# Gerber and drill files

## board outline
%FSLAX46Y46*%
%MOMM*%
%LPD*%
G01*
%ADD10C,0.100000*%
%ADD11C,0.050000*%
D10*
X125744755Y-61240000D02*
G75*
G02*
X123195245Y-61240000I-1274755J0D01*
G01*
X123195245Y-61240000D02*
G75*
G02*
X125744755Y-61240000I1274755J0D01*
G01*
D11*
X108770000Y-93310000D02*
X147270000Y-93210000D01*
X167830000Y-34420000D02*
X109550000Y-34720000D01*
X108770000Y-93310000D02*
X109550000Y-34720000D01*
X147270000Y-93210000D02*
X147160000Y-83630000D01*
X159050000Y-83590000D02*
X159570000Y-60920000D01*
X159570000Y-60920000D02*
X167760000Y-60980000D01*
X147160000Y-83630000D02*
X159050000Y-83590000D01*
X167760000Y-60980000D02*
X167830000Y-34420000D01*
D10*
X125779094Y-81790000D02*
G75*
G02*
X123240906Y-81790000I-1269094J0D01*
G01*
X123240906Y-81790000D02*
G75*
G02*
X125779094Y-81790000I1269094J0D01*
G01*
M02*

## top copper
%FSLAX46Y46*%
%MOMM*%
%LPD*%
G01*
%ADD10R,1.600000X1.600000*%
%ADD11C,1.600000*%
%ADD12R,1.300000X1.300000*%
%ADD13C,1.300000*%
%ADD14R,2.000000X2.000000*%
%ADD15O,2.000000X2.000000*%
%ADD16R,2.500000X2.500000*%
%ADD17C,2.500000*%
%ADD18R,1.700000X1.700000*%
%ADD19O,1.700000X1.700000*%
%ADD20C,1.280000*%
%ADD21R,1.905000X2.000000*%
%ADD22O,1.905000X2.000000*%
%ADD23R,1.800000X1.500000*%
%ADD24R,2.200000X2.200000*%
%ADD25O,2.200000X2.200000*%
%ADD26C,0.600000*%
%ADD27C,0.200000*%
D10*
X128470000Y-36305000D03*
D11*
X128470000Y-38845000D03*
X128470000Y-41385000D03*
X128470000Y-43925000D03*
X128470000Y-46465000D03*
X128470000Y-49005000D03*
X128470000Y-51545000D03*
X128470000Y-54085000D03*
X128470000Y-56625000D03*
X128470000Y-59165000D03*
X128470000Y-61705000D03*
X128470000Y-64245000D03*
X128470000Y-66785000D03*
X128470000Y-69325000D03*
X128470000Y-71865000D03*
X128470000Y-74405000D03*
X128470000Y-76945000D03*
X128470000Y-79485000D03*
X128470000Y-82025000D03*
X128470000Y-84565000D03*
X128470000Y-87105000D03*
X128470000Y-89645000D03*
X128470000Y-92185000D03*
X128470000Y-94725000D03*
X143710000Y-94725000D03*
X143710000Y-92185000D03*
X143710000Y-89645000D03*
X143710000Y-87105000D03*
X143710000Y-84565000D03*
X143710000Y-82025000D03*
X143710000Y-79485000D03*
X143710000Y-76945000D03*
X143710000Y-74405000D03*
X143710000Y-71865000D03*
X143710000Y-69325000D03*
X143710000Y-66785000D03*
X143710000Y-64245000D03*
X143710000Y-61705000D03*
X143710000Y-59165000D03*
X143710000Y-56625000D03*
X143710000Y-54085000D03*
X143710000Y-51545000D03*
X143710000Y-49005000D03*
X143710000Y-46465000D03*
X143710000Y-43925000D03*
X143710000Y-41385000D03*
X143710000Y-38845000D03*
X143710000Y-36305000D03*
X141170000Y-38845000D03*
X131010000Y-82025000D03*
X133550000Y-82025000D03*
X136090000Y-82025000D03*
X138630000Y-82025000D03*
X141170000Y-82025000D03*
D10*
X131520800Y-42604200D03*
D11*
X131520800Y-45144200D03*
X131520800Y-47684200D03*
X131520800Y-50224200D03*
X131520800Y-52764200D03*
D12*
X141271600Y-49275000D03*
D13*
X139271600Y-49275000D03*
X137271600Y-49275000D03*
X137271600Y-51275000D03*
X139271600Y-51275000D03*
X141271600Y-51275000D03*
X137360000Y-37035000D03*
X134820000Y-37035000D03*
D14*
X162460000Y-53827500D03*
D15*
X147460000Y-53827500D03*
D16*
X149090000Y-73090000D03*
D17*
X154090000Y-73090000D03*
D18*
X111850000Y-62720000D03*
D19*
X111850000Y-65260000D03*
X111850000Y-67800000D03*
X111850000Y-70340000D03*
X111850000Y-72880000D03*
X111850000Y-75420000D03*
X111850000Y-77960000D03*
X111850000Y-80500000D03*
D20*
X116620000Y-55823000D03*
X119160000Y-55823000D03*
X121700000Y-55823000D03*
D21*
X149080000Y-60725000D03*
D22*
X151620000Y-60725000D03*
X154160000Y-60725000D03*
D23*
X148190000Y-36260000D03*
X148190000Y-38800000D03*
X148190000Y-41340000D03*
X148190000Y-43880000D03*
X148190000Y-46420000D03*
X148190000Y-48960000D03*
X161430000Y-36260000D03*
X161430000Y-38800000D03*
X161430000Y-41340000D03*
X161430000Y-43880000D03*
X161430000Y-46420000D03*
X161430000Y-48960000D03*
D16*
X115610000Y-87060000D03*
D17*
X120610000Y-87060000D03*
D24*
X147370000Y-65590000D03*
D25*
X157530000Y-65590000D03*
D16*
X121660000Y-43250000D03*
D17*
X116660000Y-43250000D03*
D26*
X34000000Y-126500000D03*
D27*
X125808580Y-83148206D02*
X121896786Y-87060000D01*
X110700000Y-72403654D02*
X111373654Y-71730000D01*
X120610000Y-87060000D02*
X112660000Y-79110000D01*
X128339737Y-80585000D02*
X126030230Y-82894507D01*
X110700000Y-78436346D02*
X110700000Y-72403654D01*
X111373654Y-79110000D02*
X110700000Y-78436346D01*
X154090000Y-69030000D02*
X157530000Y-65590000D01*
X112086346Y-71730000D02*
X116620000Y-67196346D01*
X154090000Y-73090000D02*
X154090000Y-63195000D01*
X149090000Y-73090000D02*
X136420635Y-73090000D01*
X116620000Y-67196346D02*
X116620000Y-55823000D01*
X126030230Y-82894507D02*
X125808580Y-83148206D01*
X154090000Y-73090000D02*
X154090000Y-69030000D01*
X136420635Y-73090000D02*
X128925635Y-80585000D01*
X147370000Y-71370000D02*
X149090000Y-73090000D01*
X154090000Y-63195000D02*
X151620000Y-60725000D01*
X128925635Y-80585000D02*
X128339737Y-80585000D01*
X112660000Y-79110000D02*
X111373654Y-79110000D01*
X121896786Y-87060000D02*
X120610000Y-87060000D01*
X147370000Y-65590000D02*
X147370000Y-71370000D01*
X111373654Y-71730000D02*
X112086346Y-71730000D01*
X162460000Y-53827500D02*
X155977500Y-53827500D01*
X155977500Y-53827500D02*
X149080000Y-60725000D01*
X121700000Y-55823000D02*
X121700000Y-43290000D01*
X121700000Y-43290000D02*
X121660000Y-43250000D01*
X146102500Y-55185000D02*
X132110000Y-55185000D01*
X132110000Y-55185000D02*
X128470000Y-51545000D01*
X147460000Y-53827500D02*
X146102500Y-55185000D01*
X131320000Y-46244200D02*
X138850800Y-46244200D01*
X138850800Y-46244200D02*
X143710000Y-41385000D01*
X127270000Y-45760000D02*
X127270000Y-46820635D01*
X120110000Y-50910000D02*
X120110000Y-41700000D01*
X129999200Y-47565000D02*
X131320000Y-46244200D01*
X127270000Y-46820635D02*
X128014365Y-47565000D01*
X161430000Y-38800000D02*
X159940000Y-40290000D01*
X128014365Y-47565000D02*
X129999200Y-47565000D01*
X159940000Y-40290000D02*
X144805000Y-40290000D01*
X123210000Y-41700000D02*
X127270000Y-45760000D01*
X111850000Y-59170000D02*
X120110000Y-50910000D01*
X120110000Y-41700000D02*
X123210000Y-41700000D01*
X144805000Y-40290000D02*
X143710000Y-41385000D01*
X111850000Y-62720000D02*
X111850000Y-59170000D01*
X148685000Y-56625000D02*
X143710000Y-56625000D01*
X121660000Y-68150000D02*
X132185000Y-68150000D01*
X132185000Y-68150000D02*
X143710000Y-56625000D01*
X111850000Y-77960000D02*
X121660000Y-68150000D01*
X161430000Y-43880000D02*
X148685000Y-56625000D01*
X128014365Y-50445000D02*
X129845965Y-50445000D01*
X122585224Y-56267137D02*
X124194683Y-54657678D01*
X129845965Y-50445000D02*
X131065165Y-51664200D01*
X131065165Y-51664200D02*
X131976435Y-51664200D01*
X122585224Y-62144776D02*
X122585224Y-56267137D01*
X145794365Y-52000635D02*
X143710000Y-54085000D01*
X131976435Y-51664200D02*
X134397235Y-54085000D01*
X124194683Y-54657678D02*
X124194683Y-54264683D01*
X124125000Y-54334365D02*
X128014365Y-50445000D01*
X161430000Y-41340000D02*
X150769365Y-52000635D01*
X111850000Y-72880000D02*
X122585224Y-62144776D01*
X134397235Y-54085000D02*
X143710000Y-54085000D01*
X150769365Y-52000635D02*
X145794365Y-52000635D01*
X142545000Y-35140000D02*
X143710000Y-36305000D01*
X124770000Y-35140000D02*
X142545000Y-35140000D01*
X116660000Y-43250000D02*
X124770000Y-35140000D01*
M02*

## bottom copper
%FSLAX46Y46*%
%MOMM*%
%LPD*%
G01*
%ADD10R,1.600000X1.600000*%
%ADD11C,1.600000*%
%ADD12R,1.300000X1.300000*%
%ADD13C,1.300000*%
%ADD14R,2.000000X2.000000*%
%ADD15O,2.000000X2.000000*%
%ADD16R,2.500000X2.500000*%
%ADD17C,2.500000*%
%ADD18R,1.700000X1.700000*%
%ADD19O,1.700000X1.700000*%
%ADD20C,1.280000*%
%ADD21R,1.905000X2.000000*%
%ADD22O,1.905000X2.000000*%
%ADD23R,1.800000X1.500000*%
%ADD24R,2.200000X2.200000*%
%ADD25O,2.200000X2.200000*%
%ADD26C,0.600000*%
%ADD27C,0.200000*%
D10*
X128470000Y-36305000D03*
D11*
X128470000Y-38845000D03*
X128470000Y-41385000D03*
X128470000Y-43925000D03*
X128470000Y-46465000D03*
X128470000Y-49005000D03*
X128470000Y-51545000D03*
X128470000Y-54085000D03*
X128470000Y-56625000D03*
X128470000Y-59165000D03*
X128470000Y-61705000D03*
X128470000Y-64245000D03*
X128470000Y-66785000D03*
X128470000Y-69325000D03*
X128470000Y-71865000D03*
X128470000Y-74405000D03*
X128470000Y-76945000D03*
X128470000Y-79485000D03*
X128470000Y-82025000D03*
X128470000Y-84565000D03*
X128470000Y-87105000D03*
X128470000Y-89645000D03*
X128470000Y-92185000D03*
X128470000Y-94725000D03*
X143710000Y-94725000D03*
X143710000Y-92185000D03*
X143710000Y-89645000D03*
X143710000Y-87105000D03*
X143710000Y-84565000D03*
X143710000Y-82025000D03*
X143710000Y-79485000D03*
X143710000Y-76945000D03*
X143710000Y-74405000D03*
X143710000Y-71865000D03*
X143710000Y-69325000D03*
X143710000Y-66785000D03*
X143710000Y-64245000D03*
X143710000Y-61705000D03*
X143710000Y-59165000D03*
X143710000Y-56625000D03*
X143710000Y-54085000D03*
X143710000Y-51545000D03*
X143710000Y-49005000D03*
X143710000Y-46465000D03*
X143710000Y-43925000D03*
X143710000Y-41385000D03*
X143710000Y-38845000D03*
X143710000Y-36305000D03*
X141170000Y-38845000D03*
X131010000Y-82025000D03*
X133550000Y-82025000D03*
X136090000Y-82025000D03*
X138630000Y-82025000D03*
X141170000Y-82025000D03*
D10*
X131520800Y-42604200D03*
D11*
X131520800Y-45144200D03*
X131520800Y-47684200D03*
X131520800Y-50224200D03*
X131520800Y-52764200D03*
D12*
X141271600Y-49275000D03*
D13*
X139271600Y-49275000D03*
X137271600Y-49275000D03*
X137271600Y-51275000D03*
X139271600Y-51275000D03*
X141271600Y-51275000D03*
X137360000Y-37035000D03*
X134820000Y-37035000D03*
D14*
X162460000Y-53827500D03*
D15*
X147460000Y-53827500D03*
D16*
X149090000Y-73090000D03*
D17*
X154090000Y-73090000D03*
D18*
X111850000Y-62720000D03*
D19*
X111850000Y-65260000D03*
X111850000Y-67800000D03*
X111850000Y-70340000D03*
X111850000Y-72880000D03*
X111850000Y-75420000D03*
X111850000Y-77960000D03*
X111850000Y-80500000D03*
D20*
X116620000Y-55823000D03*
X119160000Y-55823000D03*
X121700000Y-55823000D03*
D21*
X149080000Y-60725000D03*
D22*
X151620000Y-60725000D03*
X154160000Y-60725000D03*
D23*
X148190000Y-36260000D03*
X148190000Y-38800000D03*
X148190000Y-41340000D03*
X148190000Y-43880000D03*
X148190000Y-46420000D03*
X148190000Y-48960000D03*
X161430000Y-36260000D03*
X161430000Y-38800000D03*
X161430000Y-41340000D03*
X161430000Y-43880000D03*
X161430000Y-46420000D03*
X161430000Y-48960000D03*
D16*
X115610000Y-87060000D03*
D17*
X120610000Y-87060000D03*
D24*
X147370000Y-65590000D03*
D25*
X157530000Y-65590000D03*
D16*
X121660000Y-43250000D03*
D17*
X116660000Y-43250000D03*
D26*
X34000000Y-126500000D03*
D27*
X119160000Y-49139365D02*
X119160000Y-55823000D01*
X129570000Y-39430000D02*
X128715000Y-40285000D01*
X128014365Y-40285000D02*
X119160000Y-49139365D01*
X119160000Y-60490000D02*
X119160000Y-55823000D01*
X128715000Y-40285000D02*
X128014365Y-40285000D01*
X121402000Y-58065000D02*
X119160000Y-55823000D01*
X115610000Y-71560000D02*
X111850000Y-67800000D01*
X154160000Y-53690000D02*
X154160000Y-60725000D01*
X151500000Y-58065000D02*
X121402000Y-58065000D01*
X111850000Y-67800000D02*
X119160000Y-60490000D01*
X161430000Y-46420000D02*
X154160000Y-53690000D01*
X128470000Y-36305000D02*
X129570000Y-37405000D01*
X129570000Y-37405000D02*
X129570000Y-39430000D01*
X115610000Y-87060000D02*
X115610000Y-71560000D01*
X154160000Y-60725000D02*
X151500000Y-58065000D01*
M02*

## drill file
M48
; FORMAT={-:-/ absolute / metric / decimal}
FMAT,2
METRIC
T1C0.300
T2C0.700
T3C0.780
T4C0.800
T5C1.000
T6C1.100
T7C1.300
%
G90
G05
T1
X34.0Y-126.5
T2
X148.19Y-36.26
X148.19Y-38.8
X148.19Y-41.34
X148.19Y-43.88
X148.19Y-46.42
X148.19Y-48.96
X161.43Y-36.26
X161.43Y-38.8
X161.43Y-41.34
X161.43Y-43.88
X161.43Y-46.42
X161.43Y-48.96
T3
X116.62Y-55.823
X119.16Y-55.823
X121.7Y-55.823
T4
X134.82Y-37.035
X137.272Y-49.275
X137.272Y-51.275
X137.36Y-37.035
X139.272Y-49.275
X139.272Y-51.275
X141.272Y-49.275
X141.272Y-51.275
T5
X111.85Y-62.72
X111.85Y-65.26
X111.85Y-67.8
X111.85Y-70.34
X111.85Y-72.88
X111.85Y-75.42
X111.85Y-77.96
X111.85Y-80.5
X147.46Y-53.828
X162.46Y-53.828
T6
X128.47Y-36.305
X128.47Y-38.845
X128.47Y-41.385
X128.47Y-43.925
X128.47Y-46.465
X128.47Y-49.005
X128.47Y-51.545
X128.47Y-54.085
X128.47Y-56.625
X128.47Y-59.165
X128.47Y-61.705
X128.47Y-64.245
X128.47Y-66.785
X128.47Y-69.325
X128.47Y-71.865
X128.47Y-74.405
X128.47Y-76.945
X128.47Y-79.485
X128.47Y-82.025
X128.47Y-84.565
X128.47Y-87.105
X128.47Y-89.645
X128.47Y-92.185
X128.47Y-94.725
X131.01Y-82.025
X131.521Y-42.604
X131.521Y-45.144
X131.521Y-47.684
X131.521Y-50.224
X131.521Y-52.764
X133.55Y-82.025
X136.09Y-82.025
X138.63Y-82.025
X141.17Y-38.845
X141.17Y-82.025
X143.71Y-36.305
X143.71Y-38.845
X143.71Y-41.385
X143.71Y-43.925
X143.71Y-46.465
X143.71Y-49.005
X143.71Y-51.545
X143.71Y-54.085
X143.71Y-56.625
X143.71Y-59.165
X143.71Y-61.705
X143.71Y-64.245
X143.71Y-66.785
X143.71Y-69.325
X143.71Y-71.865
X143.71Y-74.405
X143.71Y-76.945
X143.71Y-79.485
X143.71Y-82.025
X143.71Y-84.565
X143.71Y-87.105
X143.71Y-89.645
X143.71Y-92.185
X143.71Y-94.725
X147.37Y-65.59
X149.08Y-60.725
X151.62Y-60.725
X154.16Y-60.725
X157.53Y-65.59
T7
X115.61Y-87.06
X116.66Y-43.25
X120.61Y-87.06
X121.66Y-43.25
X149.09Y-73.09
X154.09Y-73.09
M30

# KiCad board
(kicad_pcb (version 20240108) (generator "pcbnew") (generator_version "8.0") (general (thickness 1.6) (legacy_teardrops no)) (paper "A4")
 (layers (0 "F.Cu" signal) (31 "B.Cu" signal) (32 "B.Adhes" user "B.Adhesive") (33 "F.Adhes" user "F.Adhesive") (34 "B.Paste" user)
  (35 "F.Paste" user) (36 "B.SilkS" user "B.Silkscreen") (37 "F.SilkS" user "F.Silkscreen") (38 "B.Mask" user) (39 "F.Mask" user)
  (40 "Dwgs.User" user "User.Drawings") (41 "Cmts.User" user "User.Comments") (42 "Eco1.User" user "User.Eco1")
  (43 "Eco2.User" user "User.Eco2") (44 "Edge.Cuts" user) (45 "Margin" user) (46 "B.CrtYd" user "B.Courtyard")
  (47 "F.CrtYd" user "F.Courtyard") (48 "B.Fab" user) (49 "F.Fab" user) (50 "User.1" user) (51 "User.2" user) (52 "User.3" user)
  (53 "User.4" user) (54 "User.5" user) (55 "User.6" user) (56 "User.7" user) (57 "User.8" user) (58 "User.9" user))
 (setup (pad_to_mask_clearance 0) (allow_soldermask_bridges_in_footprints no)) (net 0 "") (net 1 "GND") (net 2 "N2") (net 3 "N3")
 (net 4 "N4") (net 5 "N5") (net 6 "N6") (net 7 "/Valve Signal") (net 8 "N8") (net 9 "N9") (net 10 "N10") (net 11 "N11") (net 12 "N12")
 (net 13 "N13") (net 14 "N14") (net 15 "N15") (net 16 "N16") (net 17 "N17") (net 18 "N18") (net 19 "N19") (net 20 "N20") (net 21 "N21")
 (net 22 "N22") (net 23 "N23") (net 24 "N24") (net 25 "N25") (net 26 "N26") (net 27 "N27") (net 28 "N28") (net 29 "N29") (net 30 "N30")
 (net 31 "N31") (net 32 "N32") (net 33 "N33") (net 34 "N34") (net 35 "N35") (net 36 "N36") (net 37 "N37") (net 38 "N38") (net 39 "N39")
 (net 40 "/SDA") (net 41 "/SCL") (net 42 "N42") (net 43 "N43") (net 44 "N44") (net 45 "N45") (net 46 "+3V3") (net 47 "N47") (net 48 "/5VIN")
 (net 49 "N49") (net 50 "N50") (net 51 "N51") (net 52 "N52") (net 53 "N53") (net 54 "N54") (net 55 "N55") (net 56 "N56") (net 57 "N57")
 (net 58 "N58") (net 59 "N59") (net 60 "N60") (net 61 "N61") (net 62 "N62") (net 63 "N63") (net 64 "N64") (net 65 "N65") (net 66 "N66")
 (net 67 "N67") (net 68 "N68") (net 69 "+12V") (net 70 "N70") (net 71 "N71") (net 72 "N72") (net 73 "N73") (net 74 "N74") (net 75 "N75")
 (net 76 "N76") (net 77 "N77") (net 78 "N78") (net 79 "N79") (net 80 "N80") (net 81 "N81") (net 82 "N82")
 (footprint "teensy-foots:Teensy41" (layer "F.Cu") (at 136.09 65.515 -90)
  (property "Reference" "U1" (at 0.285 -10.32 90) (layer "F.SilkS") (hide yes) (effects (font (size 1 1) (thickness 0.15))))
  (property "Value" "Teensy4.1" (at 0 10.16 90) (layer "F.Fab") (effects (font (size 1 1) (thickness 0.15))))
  (pad "1" thru_hole rect (at -29.21 7.62 270) (size 1.6 1.6) (drill 1.1) (layers "*.Cu" "*.Mask") (remove_unused_layers no) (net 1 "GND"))
  (pad "2" thru_hole circle (at -26.67 7.62 270) (size 1.6 1.6) (drill 1.1) (layers "*.Cu" "*.Mask") (remove_unused_layers no) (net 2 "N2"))
  (pad "3" thru_hole circle (at -24.13 7.62 270) (size 1.6 1.6) (drill 1.1) (layers "*.Cu" "*.Mask") (remove_unused_layers no) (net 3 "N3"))
  (pad "4" thru_hole circle (at -21.59 7.62 270) (size 1.6 1.6) (drill 1.1) (layers "*.Cu" "*.Mask") (remove_unused_layers no) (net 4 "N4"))
  (pad "5" thru_hole circle (at -19.05 7.62 270) (size 1.6 1.6) (drill 1.1) (layers "*.Cu" "*.Mask") (remove_unused_layers no) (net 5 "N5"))
  (pad "6" thru_hole circle (at -16.51 7.62 270) (size 1.6 1.6) (drill 1.1) (layers "*.Cu" "*.Mask") (remove_unused_layers no) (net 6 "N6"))
  (pad "7" thru_hole circle (at -13.97 7.62 270) (size 1.6 1.6) (drill 1.1) (layers "*.Cu" "*.Mask") (remove_unused_layers no)
   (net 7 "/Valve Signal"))
  (pad "8" thru_hole circle (at -11.43 7.62 270) (size 1.6 1.6) (drill 1.1) (layers "*.Cu" "*.Mask") (remove_unused_layers no) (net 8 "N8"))
  (pad "9" thru_hole circle (at -8.89 7.62 270) (size 1.6 1.6) (drill 1.1) (layers "*.Cu" "*.Mask") (remove_unused_layers no) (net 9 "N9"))
  (pad "10" thru_hole circle (at -6.35 7.62 270) (size 1.6 1.6) (drill 1.1) (layers "*.Cu" "*.Mask") (remove_unused_layers no)
   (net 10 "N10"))
  (pad "11" thru_hole circle (at -3.81 7.62 270) (size 1.6 1.6) (drill 1.1) (layers "*.Cu" "*.Mask") (remove_unused_layers no)
   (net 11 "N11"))
  (pad "12" thru_hole circle (at -1.27 7.62 270) (size 1.6 1.6) (drill 1.1) (layers "*.Cu" "*.Mask") (remove_unused_layers no)
   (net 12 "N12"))
  (pad "13" thru_hole circle (at 1.27 7.62 270) (size 1.6 1.6) (drill 1.1) (layers "*.Cu" "*.Mask") (remove_unused_layers no) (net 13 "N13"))
  (pad "14" thru_hole circle (at 3.81 7.62 270) (size 1.6 1.6) (drill 1.1) (layers "*.Cu" "*.Mask") (remove_unused_layers no) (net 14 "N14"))
  (pad "15" thru_hole circle (at 6.35 7.62 270) (size 1.6 1.6) (drill 1.1) (layers "*.Cu" "*.Mask") (remove_unused_layers no) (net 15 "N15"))
  (pad "16" thru_hole circle (at 8.89 7.62 270) (size 1.6 1.6) (drill 1.1) (layers "*.Cu" "*.Mask") (remove_unused_layers no) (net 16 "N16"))
  (pad "17" thru_hole circle (at 11.43 7.62 270) (size 1.6 1.6) (drill 1.1) (layers "*.Cu" "*.Mask") (remove_unused_layers no)
   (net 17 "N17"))
  (pad "18" thru_hole circle (at 13.97 7.62 270) (size 1.6 1.6) (drill 1.1) (layers "*.Cu" "*.Mask") (remove_unused_layers no)
   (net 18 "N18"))
  (pad "19" thru_hole circle (at 16.51 7.62 270) (size 1.6 1.6) (drill 1.1) (layers "*.Cu" "*.Mask") (remove_unused_layers no)
   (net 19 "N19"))
  (pad "20" thru_hole circle (at 19.05 7.62 270) (size 1.6 1.6) (drill 1.1) (layers "*.Cu" "*.Mask") (remove_unused_layers no)
   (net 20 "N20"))
  (pad "21" thru_hole circle (at 21.59 7.62 270) (size 1.6 1.6) (drill 1.1) (layers "*.Cu" "*.Mask") (remove_unused_layers no)
   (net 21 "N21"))
  (pad "22" thru_hole circle (at 24.13 7.62 270) (size 1.6 1.6) (drill 1.1) (layers "*.Cu" "*.Mask") (remove_unused_layers no)
   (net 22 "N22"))
  (pad "23" thru_hole circle (at 26.67 7.62 270) (size 1.6 1.6) (drill 1.1) (layers "*.Cu" "*.Mask") (remove_unused_layers no)
   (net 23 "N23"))
  (pad "24" thru_hole circle (at 29.21 7.62 270) (size 1.6 1.6) (drill 1.1) (layers "*.Cu" "*.Mask") (remove_unused_layers no)
   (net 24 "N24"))
  (pad "25" thru_hole circle (at 29.21 -7.62 270) (size 1.6 1.6) (drill 1.1) (layers "*.Cu" "*.Mask") (remove_unused_layers no)
   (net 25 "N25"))
  (pad "26" thru_hole circle (at 26.67 -7.62 270) (size 1.6 1.6) (drill 1.1) (layers "*.Cu" "*.Mask") (remove_unused_layers no)
   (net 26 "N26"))
  (pad "27" thru_hole circle (at 24.13 -7.62 270) (size 1.6 1.6) (drill 1.1) (layers "*.Cu" "*.Mask") (remove_unused_layers no)
   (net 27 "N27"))
  (pad "28" thru_hole circle (at 21.59 -7.62 270) (size 1.6 1.6) (drill 1.1) (layers "*.Cu" "*.Mask") (remove_unused_layers no)
   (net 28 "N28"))
  (pad "29" thru_hole circle (at 19.05 -7.62 270) (size 1.6 1.6) (drill 1.1) (layers "*.Cu" "*.Mask") (remove_unused_layers no)
   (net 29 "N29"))
  (pad "30" thru_hole circle (at 16.51 -7.62 270) (size 1.6 1.6) (drill 1.1) (layers "*.Cu" "*.Mask") (remove_unused_layers no)
   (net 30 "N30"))
  (pad "31" thru_hole circle (at 13.97 -7.62 270) (size 1.6 1.6) (drill 1.1) (layers "*.Cu" "*.Mask") (remove_unused_layers no)
   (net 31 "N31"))
  (pad "32" thru_hole circle (at 11.43 -7.62 270) (size 1.6 1.6) (drill 1.1) (layers "*.Cu" "*.Mask") (remove_unused_layers no)
   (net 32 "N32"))
  (pad "33" thru_hole circle (at 8.89 -7.62 270) (size 1.6 1.6) (drill 1.1) (layers "*.Cu" "*.Mask") (remove_unused_layers no)
   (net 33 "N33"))
  (pad "34" thru_hole circle (at 6.35 -7.62 270) (size 1.6 1.6) (drill 1.1) (layers "*.Cu" "*.Mask") (remove_unused_layers no)
   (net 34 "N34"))
  (pad "35" thru_hole circle (at 3.81 -7.62 270) (size 1.6 1.6) (drill 1.1) (layers "*.Cu" "*.Mask") (remove_unused_layers no)
   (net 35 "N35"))
  (pad "36" thru_hole circle (at 1.27 -7.62 270) (size 1.6 1.6) (drill 1.1) (layers "*.Cu" "*.Mask") (remove_unused_layers no)
   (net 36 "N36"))
  (pad "37" thru_hole circle (at -1.27 -7.62 270) (size 1.6 1.6) (drill 1.1) (layers "*.Cu" "*.Mask") (remove_unused_layers no)
   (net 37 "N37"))
  (pad "38" thru_hole circle (at -3.81 -7.62 270) (size 1.6 1.6) (drill 1.1) (layers "*.Cu" "*.Mask") (remove_unused_layers no)
   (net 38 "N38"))
  (pad "39" thru_hole circle (at -6.35 -7.62 270) (size 1.6 1.6) (drill 1.1) (layers "*.Cu" "*.Mask") (remove_unused_layers no)
   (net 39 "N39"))
  (pad "40" thru_hole circle (at -8.89 -7.62 270) (size 1.6 1.6) (drill 1.1) (layers "*.Cu" "*.Mask") (remove_unused_layers no)
   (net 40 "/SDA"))
  (pad "41" thru_hole circle (at -11.43 -7.62 270) (size 1.6 1.6) (drill 1.1) (layers "*.Cu" "*.Mask") (remove_unused_layers no)
   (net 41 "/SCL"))
  (pad "42" thru_hole circle (at -13.97 -7.62 270) (size 1.6 1.6) (drill 1.1) (layers "*.Cu" "*.Mask") (remove_unused_layers no)
   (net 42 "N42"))
  (pad "43" thru_hole circle (at -16.51 -7.62 270) (size 1.6 1.6) (drill 1.1) (layers "*.Cu" "*.Mask") (remove_unused_layers no)
   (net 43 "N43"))
  (pad "44" thru_hole circle (at -19.05 -7.62 270) (size 1.6 1.6) (drill 1.1) (layers "*.Cu" "*.Mask") (remove_unused_layers no)
   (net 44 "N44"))
  (pad "45" thru_hole circle (at -21.59 -7.62 270) (size 1.6 1.6) (drill 1.1) (layers "*.Cu" "*.Mask") (remove_unused_layers no)
   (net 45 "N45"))
  (pad "46" thru_hole circle (at -24.13 -7.62 270) (size 1.6 1.6) (drill 1.1) (layers "*.Cu" "*.Mask") (remove_unused_layers no)
   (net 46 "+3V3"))
  (pad "47" thru_hole circle (at -26.67 -7.62 270) (size 1.6 1.6) (drill 1.1) (layers "*.Cu" "*.Mask") (remove_unused_layers no)
   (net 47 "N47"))
  (pad "48" thru_hole circle (at -29.21 -7.62 270) (size 1.6 1.6) (drill 1.1) (layers "*.Cu" "*.Mask") (remove_unused_layers no)
   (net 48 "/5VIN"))
  (pad "49" thru_hole circle (at -26.67 -5.08 270) (size 1.6 1.6) (drill 1.1) (layers "*.Cu" "*.Mask") (remove_unused_layers no)
   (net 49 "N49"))
  (pad "50" thru_hole circle (at 16.51 5.08 270) (size 1.6 1.6) (drill 1.1) (layers "*.Cu" "*.Mask") (remove_unused_layers no)
   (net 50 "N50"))
  (pad "51" thru_hole circle (at 16.51 2.54 270) (size 1.6 1.6) (drill 1.1) (layers "*.Cu" "*.Mask") (remove_unused_layers no)
   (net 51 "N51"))
  (pad "52" thru_hole circle (at 16.51 0 270) (size 1.6 1.6) (drill 1.1) (layers "*.Cu" "*.Mask") (remove_unused_layers no) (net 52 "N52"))
  (pad "53" thru_hole circle (at 16.51 -2.54 270) (size 1.6 1.6) (drill 1.1) (layers "*.Cu" "*.Mask") (remove_unused_layers no)
   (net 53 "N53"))
  (pad "54" thru_hole circle (at 16.51 -5.08 270) (size 1.6 1.6) (drill 1.1) (layers "*.Cu" "*.Mask") (remove_unused_layers no)
   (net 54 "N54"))
  (pad "55" thru_hole rect (at -22.9108 4.5692 270) (size 1.6 1.6) (drill 1.1) (layers "*.Cu" "*.Mask") (remove_unused_layers no)
   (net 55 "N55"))
  (pad "56" thru_hole circle (at -20.3708 4.5692 270) (size 1.6 1.6) (drill 1.1) (layers "*.Cu" "*.Mask") (remove_unused_layers no)
   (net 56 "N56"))
  (pad "57" thru_hole circle (at -17.8308 4.5692 270) (size 1.6 1.6) (drill 1.1) (layers "*.Cu" "*.Mask") (remove_unused_layers no)
   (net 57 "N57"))
  (pad "58" thru_hole circle (at -15.2908 4.5692 270) (size 1.6 1.6) (drill 1.1) (layers "*.Cu" "*.Mask") (remove_unused_layers no)
   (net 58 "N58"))
  (pad "59" thru_hole circle (at -12.7508 4.5692 270) (size 1.6 1.6) (drill 1.1) (layers "*.Cu" "*.Mask") (remove_unused_layers no)
   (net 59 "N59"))
  (pad "60" thru_hole rect (at -16.24 -5.1816 270) (size 1.3 1.3) (drill 0.8) (layers "*.Cu" "*.Mask") (remove_unused_layers no)
   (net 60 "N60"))
  (pad "61" thru_hole circle (at -16.24 -3.1816 270) (size 1.3 1.3) (drill 0.8) (layers "*.Cu" "*.Mask") (remove_unused_layers no)
   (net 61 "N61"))
  (pad "62" thru_hole circle (at -16.24 -1.1816 270) (size 1.3 1.3) (drill 0.8) (layers "*.Cu" "*.Mask") (remove_unused_layers no)
   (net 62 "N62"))
  (pad "63" thru_hole circle (at -14.24 -1.1816 270) (size 1.3 1.3) (drill 0.8) (layers "*.Cu" "*.Mask") (remove_unused_layers no)
   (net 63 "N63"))
  (pad "64" thru_hole circle (at -14.24 -3.1816 270) (size 1.3 1.3) (drill 0.8) (layers "*.Cu" "*.Mask") (remove_unused_layers no)
   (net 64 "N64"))
  (pad "65" thru_hole circle (at -14.24 -5.1816 270) (size 1.3 1.3) (drill 0.8) (layers "*.Cu" "*.Mask") (remove_unused_layers no)
   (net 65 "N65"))
  (pad "66" thru_hole circle (at -28.48 -1.27 270) (size 1.3 1.3) (drill 0.8) (layers "*.Cu" "*.Mask") (remove_unused_layers no)
   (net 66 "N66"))
  (pad "67" thru_hole circle (at -28.48 1.27 270) (size 1.3 1.3) (drill 0.8) (layers "*.Cu" "*.Mask") (remove_unused_layers no)
   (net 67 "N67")))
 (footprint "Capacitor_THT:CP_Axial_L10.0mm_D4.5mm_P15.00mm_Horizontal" (layer "F.Cu") (at 162.46 53.8275 180)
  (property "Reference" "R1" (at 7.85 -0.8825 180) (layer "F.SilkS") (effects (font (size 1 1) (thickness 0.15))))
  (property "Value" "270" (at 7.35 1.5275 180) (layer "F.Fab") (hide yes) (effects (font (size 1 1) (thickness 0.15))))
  (pad "1" thru_hole rect (at 0 0 180) (size 2 2) (drill 1) (layers "*.Cu" "*.Mask") (remove_unused_layers no) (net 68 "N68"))
  (pad "2" thru_hole oval (at 15 0 180) (size 2 2) (drill 1) (layers "*.Cu" "*.Mask") (remove_unused_layers no) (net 7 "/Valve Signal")))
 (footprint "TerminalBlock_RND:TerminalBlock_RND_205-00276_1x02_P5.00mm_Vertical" (layer "F.Cu") (at 149.09 73.09)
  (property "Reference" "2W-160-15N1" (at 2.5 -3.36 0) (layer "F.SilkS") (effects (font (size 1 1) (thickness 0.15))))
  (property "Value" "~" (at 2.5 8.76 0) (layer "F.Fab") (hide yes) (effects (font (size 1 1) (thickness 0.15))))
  (pad "1" thru_hole rect (at 0 0) (size 2.5 2.5) (drill 1.3) (layers "*.Cu" "*.Mask") (remove_unused_layers no) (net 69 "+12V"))
  (pad "2" thru_hole circle (at 5 0) (size 2.5 2.5) (drill 1.3) (layers "*.Cu" "*.Mask") (remove_unused_layers no) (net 69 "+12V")))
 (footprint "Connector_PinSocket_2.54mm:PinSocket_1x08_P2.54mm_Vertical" (layer "F.Cu") (at 111.85 62.72)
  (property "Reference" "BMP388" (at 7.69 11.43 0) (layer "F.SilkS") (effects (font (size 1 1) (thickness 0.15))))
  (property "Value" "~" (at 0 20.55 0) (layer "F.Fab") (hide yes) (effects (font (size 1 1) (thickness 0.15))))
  (pad "1" thru_hole rect (at 0 0) (size 1.7 1.7) (drill 1) (layers "*.Cu" "*.Mask") (remove_unused_layers no) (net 46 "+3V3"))
  (pad "2" thru_hole oval (at 0 2.54) (size 1.7 1.7) (drill 1) (layers "*.Cu" "*.Mask") (remove_unused_layers no) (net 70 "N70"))
  (pad "3" thru_hole oval (at 0 5.08) (size 1.7 1.7) (drill 1) (layers "*.Cu" "*.Mask") (remove_unused_layers no) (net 1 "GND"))
  (pad "4" thru_hole oval (at 0 7.62) (size 1.7 1.7) (drill 1) (layers "*.Cu" "*.Mask") (remove_unused_layers no) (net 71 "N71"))
  (pad "5" thru_hole oval (at 0 10.16) (size 1.7 1.7) (drill 1) (layers "*.Cu" "*.Mask") (remove_unused_layers no) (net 41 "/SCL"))
  (pad "6" thru_hole oval (at 0 12.7) (size 1.7 1.7) (drill 1) (layers "*.Cu" "*.Mask") (remove_unused_layers no) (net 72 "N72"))
  (pad "7" thru_hole oval (at 0 15.24) (size 1.7 1.7) (drill 1) (layers "*.Cu" "*.Mask") (remove_unused_layers no) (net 40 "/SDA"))
  (pad "8" thru_hole oval (at 0 17.78) (size 1.7 1.7) (drill 1) (layers "*.Cu" "*.Mask") (remove_unused_layers no) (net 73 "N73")))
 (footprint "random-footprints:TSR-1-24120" (layer "F.Cu") (at 119.16 55.823)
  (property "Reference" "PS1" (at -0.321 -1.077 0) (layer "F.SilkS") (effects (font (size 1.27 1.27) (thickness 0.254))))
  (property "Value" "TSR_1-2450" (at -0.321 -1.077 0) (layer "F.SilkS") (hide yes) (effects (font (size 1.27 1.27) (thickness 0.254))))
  (pad "1" thru_hole circle (at -2.54 0) (size 1.28 1.28) (drill 0.78) (layers "*.Cu" "*.Mask") (remove_unused_layers no) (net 69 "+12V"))
  (pad "2" thru_hole circle (at 0 0) (size 1.28 1.28) (drill 0.78) (layers "*.Cu" "*.Mask") (remove_unused_layers no) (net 1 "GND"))
  (pad "3" thru_hole circle (at 2.54 0) (size 1.28 1.28) (drill 0.78) (layers "*.Cu" "*.Mask") (remove_unused_layers no) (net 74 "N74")))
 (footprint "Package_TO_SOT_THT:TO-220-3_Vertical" (layer "F.Cu") (at 149.08 60.725)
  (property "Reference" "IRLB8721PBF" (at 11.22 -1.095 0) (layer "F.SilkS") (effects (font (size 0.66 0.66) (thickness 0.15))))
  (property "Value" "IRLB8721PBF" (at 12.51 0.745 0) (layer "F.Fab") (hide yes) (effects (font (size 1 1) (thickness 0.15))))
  (pad "1" thru_hole rect (at 0 0) (size 1.905 2) (drill 1.1) (layers "*.Cu" "*.Mask") (remove_unused_layers no) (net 68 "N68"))
  (pad "2" thru_hole oval (at 2.54 0) (size 1.905 2) (drill 1.1) (layers "*.Cu" "*.Mask") (remove_unused_layers no) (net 69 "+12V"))
  (pad "3" thru_hole oval (at 5.08 0) (size 1.905 2) (drill 1.1) (layers "*.Cu" "*.Mask") (remove_unused_layers no) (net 1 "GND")))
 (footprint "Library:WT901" (layer "F.Cu") (at 147.19 34.99)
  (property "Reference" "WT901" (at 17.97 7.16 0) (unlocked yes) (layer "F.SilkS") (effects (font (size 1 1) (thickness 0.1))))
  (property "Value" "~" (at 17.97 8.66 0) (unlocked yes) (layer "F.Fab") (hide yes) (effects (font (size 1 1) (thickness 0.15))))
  (pad "1" thru_hole rect (at 1 1.27) (size 1.8 1.5) (drill 0.7) (layers "*.Cu" "*.Mask") (remove_unused_layers no) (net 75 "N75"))
  (pad "2" thru_hole rect (at 1 3.81) (size 1.8 1.5) (drill 0.7) (layers "*.Cu" "*.Mask") (remove_unused_layers no) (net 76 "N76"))
  (pad "3" thru_hole rect (at 1 6.35) (size 1.8 1.5) (drill 0.7) (layers "*.Cu" "*.Mask") (remove_unused_layers no) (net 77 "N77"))
  (pad "4" thru_hole rect (at 1 8.89) (size 1.8 1.5) (drill 0.7) (layers "*.Cu" "*.Mask") (remove_unused_layers no) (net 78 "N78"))
  (pad "5" thru_hole rect (at 1 11.43) (size 1.8 1.5) (drill 0.7) (layers "*.Cu" "*.Mask") (remove_unused_layers no) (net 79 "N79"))
  (pad "6" thru_hole rect (at 1 13.97) (size 1.8 1.5) (drill 0.7) (layers "*.Cu" "*.Mask") (remove_unused_layers no) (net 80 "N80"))
  (pad "7" thru_hole rect (at 14.24 1.27) (size 1.8 1.5) (drill 0.7) (layers "*.Cu" "*.Mask") (remove_unused_layers no) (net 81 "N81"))
  (pad "8" thru_hole rect (at 14.24 3.81) (size 1.8 1.5) (drill 0.7) (layers "*.Cu" "*.Mask") (remove_unused_layers no) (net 46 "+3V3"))
  (pad "9" thru_hole rect (at 14.24 6.35) (size 1.8 1.5) (drill 0.7) (layers "*.Cu" "*.Mask") (remove_unused_layers no) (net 41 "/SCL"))
  (pad "10" thru_hole rect (at 14.24 8.89) (size 1.8 1.5) (drill 0.7) (layers "*.Cu" "*.Mask") (remove_unused_layers no) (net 40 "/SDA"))
  (pad "11" thru_hole rect (at 14.24 11.43) (size 1.8 1.5) (drill 0.7) (layers "*.Cu" "*.Mask") (remove_unused_layers no) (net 1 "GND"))
  (pad "12" thru_hole rect (at 14.24 13.97) (size 1.8 1.5) (drill 0.7) (layers "*.Cu" "*.Mask") (remove_unused_layers no) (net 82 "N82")))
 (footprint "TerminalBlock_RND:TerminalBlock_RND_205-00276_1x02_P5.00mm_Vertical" (layer "F.Cu") (at 115.61 87.06)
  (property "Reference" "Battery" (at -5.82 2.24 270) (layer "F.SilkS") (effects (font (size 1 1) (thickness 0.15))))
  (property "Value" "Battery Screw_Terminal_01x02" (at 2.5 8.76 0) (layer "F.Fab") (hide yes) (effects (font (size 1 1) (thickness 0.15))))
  (pad "1" thru_hole rect (at 0 0) (size 2.5 2.5) (drill 1.3) (layers "*.Cu" "*.Mask") (remove_unused_layers no) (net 1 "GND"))
  (pad "2" thru_hole circle (at 5 0) (size 2.5 2.5) (drill 1.3) (layers "*.Cu" "*.Mask") (remove_unused_layers no) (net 69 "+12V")))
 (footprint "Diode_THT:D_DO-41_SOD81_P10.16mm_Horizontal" (layer "F.Cu") (at 147.37 65.59)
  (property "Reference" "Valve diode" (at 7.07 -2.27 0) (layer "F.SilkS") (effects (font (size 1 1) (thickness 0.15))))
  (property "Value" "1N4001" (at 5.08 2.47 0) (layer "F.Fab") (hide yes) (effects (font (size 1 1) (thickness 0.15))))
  (pad "1" thru_hole rect (at 0 0) (size 2.2 2.2) (drill 1.1) (layers "*.Cu" "*.Mask") (remove_unused_layers no) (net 69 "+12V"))
  (pad "2" thru_hole oval (at 10.16 0) (size 2.2 2.2) (drill 1.1) (layers "*.Cu" "*.Mask") (remove_unused_layers no) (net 69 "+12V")))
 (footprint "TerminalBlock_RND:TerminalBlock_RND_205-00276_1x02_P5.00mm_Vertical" (layer "F.Cu") (at 121.66 43.25 180)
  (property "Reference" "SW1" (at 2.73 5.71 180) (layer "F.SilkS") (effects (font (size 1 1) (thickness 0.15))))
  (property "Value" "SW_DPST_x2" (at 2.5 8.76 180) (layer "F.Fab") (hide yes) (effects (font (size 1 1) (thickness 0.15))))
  (pad "1" thru_hole rect (at 0 0 180) (size 2.5 2.5) (drill 1.3) (layers "*.Cu" "*.Mask") (remove_unused_layers no) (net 74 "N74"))
  (pad "2" thru_hole circle (at 5 0 180) (size 2.5 2.5) (drill 1.3) (layers "*.Cu" "*.Mask") (remove_unused_layers no) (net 48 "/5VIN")))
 (gr_circle (center 124.47 61.24) (end 125.744755 61.24) (stroke (width 0.1) (type default)) (fill none) (layer "Edge.Cuts"))
 (gr_line (start 108.77 93.31) (end 147.27 93.21) (stroke (width 0.05) (type default)) (layer "Edge.Cuts"))
 (gr_line (start 167.83 34.42) (end 109.55 34.72) (stroke (width 0.05) (type default)) (layer "Edge.Cuts"))
 (gr_line (start 108.77 93.31) (end 109.55 34.72) (stroke (width 0.05) (type default)) (layer "Edge.Cuts"))
 (gr_line (start 147.27 93.21) (end 147.16 83.63) (stroke (width 0.05) (type default)) (layer "Edge.Cuts"))
 (gr_line (start 159.05 83.59) (end 159.57 60.92) (stroke (width 0.05) (type default)) (layer "Edge.Cuts"))
 (gr_line (start 159.57 60.92) (end 167.76 60.98) (stroke (width 0.05) (type default)) (layer "Edge.Cuts"))
 (gr_line (start 147.16 83.63) (end 159.05 83.59) (stroke (width 0.05) (type default)) (layer "Edge.Cuts"))
 (gr_line (start 167.76 60.98) (end 167.83 34.42) (stroke (width 0.05) (type default)) (layer "Edge.Cuts"))
 (gr_circle (center 124.51 81.79) (end 125.779094 81.79) (stroke (width 0.1) (type default)) (fill none) (layer "Edge.Cuts"))
 (via (at 34 126.5) (size 0.6) (drill 0.3) (layers "F.Cu" "B.Cu") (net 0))
 (segment (start 125.80858 83.148206) (end 121.896786 87.06) (width 0.2) (layer "F.Cu") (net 69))
 (segment (start 110.7 72.403654) (end 111.373654 71.73) (width 0.2) (layer "F.Cu") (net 69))
 (segment (start 120.61 87.06) (end 112.66 79.11) (width 0.2) (layer "F.Cu") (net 69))
 (segment (start 128.339737 80.585) (end 126.03023 82.894507) (width 0.2) (layer "F.Cu") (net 69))
 (segment (start 110.7 78.436346) (end 110.7 72.403654) (width 0.2) (layer "F.Cu") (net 69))
 (segment (start 111.373654 79.11) (end 110.7 78.436346) (width 0.2) (layer "F.Cu") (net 69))
 (segment (start 154.09 69.03) (end 157.53 65.59) (width 0.2) (layer "F.Cu") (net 69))
 (segment (start 112.086346 71.73) (end 116.62 67.196346) (width 0.2) (layer "F.Cu") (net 69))
 (segment (start 154.09 73.09) (end 154.09 63.195) (width 0.2) (layer "F.Cu") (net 69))
 (segment (start 149.09 73.09) (end 136.420635 73.09) (width 0.2) (layer "F.Cu") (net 69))
 (segment (start 116.62 67.196346) (end 116.62 55.823) (width 0.2) (layer "F.Cu") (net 69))
 (segment (start 126.03023 82.894507) (end 125.80858 83.148206) (width 0.2) (layer "F.Cu") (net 69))
 (segment (start 154.09 73.09) (end 154.09 69.03) (width 0.2) (layer "F.Cu") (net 69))
 (segment (start 136.420635 73.09) (end 128.925635 80.585) (width 0.2) (layer "F.Cu") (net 69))
 (segment (start 147.37 71.37) (end 149.09 73.09) (width 0.2) (layer "F.Cu") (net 69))
 (segment (start 154.09 63.195) (end 151.62 60.725) (width 0.2) (layer "F.Cu") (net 69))
 (segment (start 128.925635 80.585) (end 128.339737 80.585) (width 0.2) (layer "F.Cu") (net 69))
 (segment (start 112.66 79.11) (end 111.373654 79.11) (width 0.2) (layer "F.Cu") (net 69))
 (segment (start 121.896786 87.06) (end 120.61 87.06) (width 0.2) (layer "F.Cu") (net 69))
 (segment (start 147.37 65.59) (end 147.37 71.37) (width 0.2) (layer "F.Cu") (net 69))
 (segment (start 111.373654 71.73) (end 112.086346 71.73) (width 0.2) (layer "F.Cu") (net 69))
 (segment (start 119.16 49.139365) (end 119.16 55.823) (width 0.2) (layer "B.Cu") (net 1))
 (segment (start 129.57 39.43) (end 128.715 40.285) (width 0.2) (layer "B.Cu") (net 1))
 (segment (start 128.014365 40.285) (end 119.16 49.139365) (width 0.2) (layer "B.Cu") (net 1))
 (segment (start 119.16 60.49) (end 119.16 55.823) (width 0.2) (layer "B.Cu") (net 1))
 (segment (start 128.715 40.285) (end 128.014365 40.285) (width 0.2) (layer "B.Cu") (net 1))
 (segment (start 121.402 58.065) (end 119.16 55.823) (width 0.2) (layer "B.Cu") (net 1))
 (segment (start 115.61 71.56) (end 111.85 67.8) (width 0.2) (layer "B.Cu") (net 1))
 (segment (start 154.16 53.69) (end 154.16 60.725) (width 0.2) (layer "B.Cu") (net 1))
 (segment (start 151.5 58.065) (end 121.402 58.065) (width 0.2) (layer "B.Cu") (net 1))
 (segment (start 111.85 67.8) (end 119.16 60.49) (width 0.2) (layer "B.Cu") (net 1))
 (segment (start 161.43 46.42) (end 154.16 53.69) (width 0.2) (layer "B.Cu") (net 1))
 (segment (start 128.47 36.305) (end 129.57 37.405) (width 0.2) (layer "B.Cu") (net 1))
 (segment (start 129.57 37.405) (end 129.57 39.43) (width 0.2) (layer "B.Cu") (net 1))
 (segment (start 115.61 87.06) (end 115.61 71.56) (width 0.2) (layer "B.Cu") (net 1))
 (segment (start 154.16 60.725) (end 151.5 58.065) (width 0.2) (layer "B.Cu") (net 1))
 (segment (start 162.46 53.8275) (end 155.9775 53.8275) (width 0.2) (layer "F.Cu") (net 68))
 (segment (start 155.9775 53.8275) (end 149.08 60.725) (width 0.2) (layer "F.Cu") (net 68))
 (segment (start 121.7 55.823) (end 121.7 43.29) (width 0.2) (layer "F.Cu") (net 74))
 (segment (start 121.7 43.29) (end 121.66 43.25) (width 0.2) (layer "F.Cu") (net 74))
 (segment (start 146.1025 55.185) (end 132.11 55.185) (width 0.2) (layer "F.Cu") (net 7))
 (segment (start 132.11 55.185) (end 128.47 51.545) (width 0.2) (layer "F.Cu") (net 7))
 (segment (start 147.46 53.8275) (end 146.1025 55.185) (width 0.2) (layer "F.Cu") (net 7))
 (segment (start 131.32 46.2442) (end 138.8508 46.2442) (width 0.2) (layer "F.Cu") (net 46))
 (segment (start 138.8508 46.2442) (end 143.71 41.385) (width 0.2) (layer "F.Cu") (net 46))
 (segment (start 127.27 45.76) (end 127.27 46.820635) (width 0.2) (layer "F.Cu") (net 46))
 (segment (start 120.11 50.91) (end 120.11 41.7) (width 0.2) (layer "F.Cu") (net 46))
 (segment (start 129.9992 47.565) (end 131.32 46.2442) (width 0.2) (layer "F.Cu") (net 46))
 (segment (start 127.27 46.820635) (end 128.014365 47.565) (width 0.2) (layer "F.Cu") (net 46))
 (segment (start 161.43 38.8) (end 159.94 40.29) (width 0.2) (layer "F.Cu") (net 46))
 (segment (start 128.014365 47.565) (end 129.9992 47.565) (width 0.2) (layer "F.Cu") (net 46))
 (segment (start 159.94 40.29) (end 144.805 40.29) (width 0.2) (layer "F.Cu") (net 46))
 (segment (start 123.21 41.7) (end 127.27 45.76) (width 0.2) (layer "F.Cu") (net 46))
 (segment (start 111.85 59.17) (end 120.11 50.91) (width 0.2) (layer "F.Cu") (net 46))
 (segment (start 120.11 41.7) (end 123.21 41.7) (width 0.2) (layer "F.Cu") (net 46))
 (segment (start 144.805 40.29) (end 143.71 41.385) (width 0.2) (layer "F.Cu") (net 46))
 (segment (start 111.85 62.72) (end 111.85 59.17) (width 0.2) (layer "F.Cu") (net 46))
 (segment (start 148.685 56.625) (end 143.71 56.625) (width 0.2) (layer "F.Cu") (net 40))
 (segment (start 121.66 68.15) (end 132.185 68.15) (width 0.2) (layer "F.Cu") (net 40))
 (segment (start 132.185 68.15) (end 143.71 56.625) (width 0.2) (layer "F.Cu") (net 40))
 (segment (start 111.85 77.96) (end 121.66 68.15) (width 0.2) (layer "F.Cu") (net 40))
 (segment (start 161.43 43.88) (end 148.685 56.625) (width 0.2) (layer "F.Cu") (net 40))
 (segment (start 128.014365 50.445) (end 129.845965 50.445) (width 0.2) (layer "F.Cu") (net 41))
 (segment (start 122.585224 56.267137) (end 124.194683 54.657678) (width 0.2) (layer "F.Cu") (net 41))
 (segment (start 129.845965 50.445) (end 131.065165 51.6642) (width 0.2) (layer "F.Cu") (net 41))
 (segment (start 131.065165 51.6642) (end 131.976435 51.6642) (width 0.2) (layer "F.Cu") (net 41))
 (segment (start 122.585224 62.144776) (end 122.585224 56.267137) (width 0.2) (layer "F.Cu") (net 41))
 (segment (start 145.794365 52.000635) (end 143.71 54.085) (width 0.2) (layer "F.Cu") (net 41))
 (segment (start 131.976435 51.6642) (end 134.397235 54.085) (width 0.2) (layer "F.Cu") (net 41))
 (segment (start 124.194683 54.657678) (end 124.194683 54.264683) (width 0.2) (layer "F.Cu") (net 41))
 (segment (start 124.125 54.334365) (end 128.014365 50.445) (width 0.2) (layer "F.Cu") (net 41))
 (segment (start 161.43 41.34) (end 150.769365 52.000635) (width 0.2) (layer "F.Cu") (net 41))
 (segment (start 111.85 72.88) (end 122.585224 62.144776) (width 0.2) (layer "F.Cu") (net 41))
 (segment (start 134.397235 54.085) (end 143.71 54.085) (width 0.2) (layer "F.Cu") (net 41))
 (segment (start 150.769365 52.000635) (end 145.794365 52.000635) (width 0.2) (layer "F.Cu") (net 41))
 (segment (start 142.545 35.14) (end 143.71 36.305) (width 0.2) (layer "F.Cu") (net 48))
 (segment (start 124.77 35.14) (end 142.545 35.14) (width 0.2) (layer "F.Cu") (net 48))
 (segment (start 116.66 43.25) (end 124.77 35.14) (width 0.2) (layer "F.Cu") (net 48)))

